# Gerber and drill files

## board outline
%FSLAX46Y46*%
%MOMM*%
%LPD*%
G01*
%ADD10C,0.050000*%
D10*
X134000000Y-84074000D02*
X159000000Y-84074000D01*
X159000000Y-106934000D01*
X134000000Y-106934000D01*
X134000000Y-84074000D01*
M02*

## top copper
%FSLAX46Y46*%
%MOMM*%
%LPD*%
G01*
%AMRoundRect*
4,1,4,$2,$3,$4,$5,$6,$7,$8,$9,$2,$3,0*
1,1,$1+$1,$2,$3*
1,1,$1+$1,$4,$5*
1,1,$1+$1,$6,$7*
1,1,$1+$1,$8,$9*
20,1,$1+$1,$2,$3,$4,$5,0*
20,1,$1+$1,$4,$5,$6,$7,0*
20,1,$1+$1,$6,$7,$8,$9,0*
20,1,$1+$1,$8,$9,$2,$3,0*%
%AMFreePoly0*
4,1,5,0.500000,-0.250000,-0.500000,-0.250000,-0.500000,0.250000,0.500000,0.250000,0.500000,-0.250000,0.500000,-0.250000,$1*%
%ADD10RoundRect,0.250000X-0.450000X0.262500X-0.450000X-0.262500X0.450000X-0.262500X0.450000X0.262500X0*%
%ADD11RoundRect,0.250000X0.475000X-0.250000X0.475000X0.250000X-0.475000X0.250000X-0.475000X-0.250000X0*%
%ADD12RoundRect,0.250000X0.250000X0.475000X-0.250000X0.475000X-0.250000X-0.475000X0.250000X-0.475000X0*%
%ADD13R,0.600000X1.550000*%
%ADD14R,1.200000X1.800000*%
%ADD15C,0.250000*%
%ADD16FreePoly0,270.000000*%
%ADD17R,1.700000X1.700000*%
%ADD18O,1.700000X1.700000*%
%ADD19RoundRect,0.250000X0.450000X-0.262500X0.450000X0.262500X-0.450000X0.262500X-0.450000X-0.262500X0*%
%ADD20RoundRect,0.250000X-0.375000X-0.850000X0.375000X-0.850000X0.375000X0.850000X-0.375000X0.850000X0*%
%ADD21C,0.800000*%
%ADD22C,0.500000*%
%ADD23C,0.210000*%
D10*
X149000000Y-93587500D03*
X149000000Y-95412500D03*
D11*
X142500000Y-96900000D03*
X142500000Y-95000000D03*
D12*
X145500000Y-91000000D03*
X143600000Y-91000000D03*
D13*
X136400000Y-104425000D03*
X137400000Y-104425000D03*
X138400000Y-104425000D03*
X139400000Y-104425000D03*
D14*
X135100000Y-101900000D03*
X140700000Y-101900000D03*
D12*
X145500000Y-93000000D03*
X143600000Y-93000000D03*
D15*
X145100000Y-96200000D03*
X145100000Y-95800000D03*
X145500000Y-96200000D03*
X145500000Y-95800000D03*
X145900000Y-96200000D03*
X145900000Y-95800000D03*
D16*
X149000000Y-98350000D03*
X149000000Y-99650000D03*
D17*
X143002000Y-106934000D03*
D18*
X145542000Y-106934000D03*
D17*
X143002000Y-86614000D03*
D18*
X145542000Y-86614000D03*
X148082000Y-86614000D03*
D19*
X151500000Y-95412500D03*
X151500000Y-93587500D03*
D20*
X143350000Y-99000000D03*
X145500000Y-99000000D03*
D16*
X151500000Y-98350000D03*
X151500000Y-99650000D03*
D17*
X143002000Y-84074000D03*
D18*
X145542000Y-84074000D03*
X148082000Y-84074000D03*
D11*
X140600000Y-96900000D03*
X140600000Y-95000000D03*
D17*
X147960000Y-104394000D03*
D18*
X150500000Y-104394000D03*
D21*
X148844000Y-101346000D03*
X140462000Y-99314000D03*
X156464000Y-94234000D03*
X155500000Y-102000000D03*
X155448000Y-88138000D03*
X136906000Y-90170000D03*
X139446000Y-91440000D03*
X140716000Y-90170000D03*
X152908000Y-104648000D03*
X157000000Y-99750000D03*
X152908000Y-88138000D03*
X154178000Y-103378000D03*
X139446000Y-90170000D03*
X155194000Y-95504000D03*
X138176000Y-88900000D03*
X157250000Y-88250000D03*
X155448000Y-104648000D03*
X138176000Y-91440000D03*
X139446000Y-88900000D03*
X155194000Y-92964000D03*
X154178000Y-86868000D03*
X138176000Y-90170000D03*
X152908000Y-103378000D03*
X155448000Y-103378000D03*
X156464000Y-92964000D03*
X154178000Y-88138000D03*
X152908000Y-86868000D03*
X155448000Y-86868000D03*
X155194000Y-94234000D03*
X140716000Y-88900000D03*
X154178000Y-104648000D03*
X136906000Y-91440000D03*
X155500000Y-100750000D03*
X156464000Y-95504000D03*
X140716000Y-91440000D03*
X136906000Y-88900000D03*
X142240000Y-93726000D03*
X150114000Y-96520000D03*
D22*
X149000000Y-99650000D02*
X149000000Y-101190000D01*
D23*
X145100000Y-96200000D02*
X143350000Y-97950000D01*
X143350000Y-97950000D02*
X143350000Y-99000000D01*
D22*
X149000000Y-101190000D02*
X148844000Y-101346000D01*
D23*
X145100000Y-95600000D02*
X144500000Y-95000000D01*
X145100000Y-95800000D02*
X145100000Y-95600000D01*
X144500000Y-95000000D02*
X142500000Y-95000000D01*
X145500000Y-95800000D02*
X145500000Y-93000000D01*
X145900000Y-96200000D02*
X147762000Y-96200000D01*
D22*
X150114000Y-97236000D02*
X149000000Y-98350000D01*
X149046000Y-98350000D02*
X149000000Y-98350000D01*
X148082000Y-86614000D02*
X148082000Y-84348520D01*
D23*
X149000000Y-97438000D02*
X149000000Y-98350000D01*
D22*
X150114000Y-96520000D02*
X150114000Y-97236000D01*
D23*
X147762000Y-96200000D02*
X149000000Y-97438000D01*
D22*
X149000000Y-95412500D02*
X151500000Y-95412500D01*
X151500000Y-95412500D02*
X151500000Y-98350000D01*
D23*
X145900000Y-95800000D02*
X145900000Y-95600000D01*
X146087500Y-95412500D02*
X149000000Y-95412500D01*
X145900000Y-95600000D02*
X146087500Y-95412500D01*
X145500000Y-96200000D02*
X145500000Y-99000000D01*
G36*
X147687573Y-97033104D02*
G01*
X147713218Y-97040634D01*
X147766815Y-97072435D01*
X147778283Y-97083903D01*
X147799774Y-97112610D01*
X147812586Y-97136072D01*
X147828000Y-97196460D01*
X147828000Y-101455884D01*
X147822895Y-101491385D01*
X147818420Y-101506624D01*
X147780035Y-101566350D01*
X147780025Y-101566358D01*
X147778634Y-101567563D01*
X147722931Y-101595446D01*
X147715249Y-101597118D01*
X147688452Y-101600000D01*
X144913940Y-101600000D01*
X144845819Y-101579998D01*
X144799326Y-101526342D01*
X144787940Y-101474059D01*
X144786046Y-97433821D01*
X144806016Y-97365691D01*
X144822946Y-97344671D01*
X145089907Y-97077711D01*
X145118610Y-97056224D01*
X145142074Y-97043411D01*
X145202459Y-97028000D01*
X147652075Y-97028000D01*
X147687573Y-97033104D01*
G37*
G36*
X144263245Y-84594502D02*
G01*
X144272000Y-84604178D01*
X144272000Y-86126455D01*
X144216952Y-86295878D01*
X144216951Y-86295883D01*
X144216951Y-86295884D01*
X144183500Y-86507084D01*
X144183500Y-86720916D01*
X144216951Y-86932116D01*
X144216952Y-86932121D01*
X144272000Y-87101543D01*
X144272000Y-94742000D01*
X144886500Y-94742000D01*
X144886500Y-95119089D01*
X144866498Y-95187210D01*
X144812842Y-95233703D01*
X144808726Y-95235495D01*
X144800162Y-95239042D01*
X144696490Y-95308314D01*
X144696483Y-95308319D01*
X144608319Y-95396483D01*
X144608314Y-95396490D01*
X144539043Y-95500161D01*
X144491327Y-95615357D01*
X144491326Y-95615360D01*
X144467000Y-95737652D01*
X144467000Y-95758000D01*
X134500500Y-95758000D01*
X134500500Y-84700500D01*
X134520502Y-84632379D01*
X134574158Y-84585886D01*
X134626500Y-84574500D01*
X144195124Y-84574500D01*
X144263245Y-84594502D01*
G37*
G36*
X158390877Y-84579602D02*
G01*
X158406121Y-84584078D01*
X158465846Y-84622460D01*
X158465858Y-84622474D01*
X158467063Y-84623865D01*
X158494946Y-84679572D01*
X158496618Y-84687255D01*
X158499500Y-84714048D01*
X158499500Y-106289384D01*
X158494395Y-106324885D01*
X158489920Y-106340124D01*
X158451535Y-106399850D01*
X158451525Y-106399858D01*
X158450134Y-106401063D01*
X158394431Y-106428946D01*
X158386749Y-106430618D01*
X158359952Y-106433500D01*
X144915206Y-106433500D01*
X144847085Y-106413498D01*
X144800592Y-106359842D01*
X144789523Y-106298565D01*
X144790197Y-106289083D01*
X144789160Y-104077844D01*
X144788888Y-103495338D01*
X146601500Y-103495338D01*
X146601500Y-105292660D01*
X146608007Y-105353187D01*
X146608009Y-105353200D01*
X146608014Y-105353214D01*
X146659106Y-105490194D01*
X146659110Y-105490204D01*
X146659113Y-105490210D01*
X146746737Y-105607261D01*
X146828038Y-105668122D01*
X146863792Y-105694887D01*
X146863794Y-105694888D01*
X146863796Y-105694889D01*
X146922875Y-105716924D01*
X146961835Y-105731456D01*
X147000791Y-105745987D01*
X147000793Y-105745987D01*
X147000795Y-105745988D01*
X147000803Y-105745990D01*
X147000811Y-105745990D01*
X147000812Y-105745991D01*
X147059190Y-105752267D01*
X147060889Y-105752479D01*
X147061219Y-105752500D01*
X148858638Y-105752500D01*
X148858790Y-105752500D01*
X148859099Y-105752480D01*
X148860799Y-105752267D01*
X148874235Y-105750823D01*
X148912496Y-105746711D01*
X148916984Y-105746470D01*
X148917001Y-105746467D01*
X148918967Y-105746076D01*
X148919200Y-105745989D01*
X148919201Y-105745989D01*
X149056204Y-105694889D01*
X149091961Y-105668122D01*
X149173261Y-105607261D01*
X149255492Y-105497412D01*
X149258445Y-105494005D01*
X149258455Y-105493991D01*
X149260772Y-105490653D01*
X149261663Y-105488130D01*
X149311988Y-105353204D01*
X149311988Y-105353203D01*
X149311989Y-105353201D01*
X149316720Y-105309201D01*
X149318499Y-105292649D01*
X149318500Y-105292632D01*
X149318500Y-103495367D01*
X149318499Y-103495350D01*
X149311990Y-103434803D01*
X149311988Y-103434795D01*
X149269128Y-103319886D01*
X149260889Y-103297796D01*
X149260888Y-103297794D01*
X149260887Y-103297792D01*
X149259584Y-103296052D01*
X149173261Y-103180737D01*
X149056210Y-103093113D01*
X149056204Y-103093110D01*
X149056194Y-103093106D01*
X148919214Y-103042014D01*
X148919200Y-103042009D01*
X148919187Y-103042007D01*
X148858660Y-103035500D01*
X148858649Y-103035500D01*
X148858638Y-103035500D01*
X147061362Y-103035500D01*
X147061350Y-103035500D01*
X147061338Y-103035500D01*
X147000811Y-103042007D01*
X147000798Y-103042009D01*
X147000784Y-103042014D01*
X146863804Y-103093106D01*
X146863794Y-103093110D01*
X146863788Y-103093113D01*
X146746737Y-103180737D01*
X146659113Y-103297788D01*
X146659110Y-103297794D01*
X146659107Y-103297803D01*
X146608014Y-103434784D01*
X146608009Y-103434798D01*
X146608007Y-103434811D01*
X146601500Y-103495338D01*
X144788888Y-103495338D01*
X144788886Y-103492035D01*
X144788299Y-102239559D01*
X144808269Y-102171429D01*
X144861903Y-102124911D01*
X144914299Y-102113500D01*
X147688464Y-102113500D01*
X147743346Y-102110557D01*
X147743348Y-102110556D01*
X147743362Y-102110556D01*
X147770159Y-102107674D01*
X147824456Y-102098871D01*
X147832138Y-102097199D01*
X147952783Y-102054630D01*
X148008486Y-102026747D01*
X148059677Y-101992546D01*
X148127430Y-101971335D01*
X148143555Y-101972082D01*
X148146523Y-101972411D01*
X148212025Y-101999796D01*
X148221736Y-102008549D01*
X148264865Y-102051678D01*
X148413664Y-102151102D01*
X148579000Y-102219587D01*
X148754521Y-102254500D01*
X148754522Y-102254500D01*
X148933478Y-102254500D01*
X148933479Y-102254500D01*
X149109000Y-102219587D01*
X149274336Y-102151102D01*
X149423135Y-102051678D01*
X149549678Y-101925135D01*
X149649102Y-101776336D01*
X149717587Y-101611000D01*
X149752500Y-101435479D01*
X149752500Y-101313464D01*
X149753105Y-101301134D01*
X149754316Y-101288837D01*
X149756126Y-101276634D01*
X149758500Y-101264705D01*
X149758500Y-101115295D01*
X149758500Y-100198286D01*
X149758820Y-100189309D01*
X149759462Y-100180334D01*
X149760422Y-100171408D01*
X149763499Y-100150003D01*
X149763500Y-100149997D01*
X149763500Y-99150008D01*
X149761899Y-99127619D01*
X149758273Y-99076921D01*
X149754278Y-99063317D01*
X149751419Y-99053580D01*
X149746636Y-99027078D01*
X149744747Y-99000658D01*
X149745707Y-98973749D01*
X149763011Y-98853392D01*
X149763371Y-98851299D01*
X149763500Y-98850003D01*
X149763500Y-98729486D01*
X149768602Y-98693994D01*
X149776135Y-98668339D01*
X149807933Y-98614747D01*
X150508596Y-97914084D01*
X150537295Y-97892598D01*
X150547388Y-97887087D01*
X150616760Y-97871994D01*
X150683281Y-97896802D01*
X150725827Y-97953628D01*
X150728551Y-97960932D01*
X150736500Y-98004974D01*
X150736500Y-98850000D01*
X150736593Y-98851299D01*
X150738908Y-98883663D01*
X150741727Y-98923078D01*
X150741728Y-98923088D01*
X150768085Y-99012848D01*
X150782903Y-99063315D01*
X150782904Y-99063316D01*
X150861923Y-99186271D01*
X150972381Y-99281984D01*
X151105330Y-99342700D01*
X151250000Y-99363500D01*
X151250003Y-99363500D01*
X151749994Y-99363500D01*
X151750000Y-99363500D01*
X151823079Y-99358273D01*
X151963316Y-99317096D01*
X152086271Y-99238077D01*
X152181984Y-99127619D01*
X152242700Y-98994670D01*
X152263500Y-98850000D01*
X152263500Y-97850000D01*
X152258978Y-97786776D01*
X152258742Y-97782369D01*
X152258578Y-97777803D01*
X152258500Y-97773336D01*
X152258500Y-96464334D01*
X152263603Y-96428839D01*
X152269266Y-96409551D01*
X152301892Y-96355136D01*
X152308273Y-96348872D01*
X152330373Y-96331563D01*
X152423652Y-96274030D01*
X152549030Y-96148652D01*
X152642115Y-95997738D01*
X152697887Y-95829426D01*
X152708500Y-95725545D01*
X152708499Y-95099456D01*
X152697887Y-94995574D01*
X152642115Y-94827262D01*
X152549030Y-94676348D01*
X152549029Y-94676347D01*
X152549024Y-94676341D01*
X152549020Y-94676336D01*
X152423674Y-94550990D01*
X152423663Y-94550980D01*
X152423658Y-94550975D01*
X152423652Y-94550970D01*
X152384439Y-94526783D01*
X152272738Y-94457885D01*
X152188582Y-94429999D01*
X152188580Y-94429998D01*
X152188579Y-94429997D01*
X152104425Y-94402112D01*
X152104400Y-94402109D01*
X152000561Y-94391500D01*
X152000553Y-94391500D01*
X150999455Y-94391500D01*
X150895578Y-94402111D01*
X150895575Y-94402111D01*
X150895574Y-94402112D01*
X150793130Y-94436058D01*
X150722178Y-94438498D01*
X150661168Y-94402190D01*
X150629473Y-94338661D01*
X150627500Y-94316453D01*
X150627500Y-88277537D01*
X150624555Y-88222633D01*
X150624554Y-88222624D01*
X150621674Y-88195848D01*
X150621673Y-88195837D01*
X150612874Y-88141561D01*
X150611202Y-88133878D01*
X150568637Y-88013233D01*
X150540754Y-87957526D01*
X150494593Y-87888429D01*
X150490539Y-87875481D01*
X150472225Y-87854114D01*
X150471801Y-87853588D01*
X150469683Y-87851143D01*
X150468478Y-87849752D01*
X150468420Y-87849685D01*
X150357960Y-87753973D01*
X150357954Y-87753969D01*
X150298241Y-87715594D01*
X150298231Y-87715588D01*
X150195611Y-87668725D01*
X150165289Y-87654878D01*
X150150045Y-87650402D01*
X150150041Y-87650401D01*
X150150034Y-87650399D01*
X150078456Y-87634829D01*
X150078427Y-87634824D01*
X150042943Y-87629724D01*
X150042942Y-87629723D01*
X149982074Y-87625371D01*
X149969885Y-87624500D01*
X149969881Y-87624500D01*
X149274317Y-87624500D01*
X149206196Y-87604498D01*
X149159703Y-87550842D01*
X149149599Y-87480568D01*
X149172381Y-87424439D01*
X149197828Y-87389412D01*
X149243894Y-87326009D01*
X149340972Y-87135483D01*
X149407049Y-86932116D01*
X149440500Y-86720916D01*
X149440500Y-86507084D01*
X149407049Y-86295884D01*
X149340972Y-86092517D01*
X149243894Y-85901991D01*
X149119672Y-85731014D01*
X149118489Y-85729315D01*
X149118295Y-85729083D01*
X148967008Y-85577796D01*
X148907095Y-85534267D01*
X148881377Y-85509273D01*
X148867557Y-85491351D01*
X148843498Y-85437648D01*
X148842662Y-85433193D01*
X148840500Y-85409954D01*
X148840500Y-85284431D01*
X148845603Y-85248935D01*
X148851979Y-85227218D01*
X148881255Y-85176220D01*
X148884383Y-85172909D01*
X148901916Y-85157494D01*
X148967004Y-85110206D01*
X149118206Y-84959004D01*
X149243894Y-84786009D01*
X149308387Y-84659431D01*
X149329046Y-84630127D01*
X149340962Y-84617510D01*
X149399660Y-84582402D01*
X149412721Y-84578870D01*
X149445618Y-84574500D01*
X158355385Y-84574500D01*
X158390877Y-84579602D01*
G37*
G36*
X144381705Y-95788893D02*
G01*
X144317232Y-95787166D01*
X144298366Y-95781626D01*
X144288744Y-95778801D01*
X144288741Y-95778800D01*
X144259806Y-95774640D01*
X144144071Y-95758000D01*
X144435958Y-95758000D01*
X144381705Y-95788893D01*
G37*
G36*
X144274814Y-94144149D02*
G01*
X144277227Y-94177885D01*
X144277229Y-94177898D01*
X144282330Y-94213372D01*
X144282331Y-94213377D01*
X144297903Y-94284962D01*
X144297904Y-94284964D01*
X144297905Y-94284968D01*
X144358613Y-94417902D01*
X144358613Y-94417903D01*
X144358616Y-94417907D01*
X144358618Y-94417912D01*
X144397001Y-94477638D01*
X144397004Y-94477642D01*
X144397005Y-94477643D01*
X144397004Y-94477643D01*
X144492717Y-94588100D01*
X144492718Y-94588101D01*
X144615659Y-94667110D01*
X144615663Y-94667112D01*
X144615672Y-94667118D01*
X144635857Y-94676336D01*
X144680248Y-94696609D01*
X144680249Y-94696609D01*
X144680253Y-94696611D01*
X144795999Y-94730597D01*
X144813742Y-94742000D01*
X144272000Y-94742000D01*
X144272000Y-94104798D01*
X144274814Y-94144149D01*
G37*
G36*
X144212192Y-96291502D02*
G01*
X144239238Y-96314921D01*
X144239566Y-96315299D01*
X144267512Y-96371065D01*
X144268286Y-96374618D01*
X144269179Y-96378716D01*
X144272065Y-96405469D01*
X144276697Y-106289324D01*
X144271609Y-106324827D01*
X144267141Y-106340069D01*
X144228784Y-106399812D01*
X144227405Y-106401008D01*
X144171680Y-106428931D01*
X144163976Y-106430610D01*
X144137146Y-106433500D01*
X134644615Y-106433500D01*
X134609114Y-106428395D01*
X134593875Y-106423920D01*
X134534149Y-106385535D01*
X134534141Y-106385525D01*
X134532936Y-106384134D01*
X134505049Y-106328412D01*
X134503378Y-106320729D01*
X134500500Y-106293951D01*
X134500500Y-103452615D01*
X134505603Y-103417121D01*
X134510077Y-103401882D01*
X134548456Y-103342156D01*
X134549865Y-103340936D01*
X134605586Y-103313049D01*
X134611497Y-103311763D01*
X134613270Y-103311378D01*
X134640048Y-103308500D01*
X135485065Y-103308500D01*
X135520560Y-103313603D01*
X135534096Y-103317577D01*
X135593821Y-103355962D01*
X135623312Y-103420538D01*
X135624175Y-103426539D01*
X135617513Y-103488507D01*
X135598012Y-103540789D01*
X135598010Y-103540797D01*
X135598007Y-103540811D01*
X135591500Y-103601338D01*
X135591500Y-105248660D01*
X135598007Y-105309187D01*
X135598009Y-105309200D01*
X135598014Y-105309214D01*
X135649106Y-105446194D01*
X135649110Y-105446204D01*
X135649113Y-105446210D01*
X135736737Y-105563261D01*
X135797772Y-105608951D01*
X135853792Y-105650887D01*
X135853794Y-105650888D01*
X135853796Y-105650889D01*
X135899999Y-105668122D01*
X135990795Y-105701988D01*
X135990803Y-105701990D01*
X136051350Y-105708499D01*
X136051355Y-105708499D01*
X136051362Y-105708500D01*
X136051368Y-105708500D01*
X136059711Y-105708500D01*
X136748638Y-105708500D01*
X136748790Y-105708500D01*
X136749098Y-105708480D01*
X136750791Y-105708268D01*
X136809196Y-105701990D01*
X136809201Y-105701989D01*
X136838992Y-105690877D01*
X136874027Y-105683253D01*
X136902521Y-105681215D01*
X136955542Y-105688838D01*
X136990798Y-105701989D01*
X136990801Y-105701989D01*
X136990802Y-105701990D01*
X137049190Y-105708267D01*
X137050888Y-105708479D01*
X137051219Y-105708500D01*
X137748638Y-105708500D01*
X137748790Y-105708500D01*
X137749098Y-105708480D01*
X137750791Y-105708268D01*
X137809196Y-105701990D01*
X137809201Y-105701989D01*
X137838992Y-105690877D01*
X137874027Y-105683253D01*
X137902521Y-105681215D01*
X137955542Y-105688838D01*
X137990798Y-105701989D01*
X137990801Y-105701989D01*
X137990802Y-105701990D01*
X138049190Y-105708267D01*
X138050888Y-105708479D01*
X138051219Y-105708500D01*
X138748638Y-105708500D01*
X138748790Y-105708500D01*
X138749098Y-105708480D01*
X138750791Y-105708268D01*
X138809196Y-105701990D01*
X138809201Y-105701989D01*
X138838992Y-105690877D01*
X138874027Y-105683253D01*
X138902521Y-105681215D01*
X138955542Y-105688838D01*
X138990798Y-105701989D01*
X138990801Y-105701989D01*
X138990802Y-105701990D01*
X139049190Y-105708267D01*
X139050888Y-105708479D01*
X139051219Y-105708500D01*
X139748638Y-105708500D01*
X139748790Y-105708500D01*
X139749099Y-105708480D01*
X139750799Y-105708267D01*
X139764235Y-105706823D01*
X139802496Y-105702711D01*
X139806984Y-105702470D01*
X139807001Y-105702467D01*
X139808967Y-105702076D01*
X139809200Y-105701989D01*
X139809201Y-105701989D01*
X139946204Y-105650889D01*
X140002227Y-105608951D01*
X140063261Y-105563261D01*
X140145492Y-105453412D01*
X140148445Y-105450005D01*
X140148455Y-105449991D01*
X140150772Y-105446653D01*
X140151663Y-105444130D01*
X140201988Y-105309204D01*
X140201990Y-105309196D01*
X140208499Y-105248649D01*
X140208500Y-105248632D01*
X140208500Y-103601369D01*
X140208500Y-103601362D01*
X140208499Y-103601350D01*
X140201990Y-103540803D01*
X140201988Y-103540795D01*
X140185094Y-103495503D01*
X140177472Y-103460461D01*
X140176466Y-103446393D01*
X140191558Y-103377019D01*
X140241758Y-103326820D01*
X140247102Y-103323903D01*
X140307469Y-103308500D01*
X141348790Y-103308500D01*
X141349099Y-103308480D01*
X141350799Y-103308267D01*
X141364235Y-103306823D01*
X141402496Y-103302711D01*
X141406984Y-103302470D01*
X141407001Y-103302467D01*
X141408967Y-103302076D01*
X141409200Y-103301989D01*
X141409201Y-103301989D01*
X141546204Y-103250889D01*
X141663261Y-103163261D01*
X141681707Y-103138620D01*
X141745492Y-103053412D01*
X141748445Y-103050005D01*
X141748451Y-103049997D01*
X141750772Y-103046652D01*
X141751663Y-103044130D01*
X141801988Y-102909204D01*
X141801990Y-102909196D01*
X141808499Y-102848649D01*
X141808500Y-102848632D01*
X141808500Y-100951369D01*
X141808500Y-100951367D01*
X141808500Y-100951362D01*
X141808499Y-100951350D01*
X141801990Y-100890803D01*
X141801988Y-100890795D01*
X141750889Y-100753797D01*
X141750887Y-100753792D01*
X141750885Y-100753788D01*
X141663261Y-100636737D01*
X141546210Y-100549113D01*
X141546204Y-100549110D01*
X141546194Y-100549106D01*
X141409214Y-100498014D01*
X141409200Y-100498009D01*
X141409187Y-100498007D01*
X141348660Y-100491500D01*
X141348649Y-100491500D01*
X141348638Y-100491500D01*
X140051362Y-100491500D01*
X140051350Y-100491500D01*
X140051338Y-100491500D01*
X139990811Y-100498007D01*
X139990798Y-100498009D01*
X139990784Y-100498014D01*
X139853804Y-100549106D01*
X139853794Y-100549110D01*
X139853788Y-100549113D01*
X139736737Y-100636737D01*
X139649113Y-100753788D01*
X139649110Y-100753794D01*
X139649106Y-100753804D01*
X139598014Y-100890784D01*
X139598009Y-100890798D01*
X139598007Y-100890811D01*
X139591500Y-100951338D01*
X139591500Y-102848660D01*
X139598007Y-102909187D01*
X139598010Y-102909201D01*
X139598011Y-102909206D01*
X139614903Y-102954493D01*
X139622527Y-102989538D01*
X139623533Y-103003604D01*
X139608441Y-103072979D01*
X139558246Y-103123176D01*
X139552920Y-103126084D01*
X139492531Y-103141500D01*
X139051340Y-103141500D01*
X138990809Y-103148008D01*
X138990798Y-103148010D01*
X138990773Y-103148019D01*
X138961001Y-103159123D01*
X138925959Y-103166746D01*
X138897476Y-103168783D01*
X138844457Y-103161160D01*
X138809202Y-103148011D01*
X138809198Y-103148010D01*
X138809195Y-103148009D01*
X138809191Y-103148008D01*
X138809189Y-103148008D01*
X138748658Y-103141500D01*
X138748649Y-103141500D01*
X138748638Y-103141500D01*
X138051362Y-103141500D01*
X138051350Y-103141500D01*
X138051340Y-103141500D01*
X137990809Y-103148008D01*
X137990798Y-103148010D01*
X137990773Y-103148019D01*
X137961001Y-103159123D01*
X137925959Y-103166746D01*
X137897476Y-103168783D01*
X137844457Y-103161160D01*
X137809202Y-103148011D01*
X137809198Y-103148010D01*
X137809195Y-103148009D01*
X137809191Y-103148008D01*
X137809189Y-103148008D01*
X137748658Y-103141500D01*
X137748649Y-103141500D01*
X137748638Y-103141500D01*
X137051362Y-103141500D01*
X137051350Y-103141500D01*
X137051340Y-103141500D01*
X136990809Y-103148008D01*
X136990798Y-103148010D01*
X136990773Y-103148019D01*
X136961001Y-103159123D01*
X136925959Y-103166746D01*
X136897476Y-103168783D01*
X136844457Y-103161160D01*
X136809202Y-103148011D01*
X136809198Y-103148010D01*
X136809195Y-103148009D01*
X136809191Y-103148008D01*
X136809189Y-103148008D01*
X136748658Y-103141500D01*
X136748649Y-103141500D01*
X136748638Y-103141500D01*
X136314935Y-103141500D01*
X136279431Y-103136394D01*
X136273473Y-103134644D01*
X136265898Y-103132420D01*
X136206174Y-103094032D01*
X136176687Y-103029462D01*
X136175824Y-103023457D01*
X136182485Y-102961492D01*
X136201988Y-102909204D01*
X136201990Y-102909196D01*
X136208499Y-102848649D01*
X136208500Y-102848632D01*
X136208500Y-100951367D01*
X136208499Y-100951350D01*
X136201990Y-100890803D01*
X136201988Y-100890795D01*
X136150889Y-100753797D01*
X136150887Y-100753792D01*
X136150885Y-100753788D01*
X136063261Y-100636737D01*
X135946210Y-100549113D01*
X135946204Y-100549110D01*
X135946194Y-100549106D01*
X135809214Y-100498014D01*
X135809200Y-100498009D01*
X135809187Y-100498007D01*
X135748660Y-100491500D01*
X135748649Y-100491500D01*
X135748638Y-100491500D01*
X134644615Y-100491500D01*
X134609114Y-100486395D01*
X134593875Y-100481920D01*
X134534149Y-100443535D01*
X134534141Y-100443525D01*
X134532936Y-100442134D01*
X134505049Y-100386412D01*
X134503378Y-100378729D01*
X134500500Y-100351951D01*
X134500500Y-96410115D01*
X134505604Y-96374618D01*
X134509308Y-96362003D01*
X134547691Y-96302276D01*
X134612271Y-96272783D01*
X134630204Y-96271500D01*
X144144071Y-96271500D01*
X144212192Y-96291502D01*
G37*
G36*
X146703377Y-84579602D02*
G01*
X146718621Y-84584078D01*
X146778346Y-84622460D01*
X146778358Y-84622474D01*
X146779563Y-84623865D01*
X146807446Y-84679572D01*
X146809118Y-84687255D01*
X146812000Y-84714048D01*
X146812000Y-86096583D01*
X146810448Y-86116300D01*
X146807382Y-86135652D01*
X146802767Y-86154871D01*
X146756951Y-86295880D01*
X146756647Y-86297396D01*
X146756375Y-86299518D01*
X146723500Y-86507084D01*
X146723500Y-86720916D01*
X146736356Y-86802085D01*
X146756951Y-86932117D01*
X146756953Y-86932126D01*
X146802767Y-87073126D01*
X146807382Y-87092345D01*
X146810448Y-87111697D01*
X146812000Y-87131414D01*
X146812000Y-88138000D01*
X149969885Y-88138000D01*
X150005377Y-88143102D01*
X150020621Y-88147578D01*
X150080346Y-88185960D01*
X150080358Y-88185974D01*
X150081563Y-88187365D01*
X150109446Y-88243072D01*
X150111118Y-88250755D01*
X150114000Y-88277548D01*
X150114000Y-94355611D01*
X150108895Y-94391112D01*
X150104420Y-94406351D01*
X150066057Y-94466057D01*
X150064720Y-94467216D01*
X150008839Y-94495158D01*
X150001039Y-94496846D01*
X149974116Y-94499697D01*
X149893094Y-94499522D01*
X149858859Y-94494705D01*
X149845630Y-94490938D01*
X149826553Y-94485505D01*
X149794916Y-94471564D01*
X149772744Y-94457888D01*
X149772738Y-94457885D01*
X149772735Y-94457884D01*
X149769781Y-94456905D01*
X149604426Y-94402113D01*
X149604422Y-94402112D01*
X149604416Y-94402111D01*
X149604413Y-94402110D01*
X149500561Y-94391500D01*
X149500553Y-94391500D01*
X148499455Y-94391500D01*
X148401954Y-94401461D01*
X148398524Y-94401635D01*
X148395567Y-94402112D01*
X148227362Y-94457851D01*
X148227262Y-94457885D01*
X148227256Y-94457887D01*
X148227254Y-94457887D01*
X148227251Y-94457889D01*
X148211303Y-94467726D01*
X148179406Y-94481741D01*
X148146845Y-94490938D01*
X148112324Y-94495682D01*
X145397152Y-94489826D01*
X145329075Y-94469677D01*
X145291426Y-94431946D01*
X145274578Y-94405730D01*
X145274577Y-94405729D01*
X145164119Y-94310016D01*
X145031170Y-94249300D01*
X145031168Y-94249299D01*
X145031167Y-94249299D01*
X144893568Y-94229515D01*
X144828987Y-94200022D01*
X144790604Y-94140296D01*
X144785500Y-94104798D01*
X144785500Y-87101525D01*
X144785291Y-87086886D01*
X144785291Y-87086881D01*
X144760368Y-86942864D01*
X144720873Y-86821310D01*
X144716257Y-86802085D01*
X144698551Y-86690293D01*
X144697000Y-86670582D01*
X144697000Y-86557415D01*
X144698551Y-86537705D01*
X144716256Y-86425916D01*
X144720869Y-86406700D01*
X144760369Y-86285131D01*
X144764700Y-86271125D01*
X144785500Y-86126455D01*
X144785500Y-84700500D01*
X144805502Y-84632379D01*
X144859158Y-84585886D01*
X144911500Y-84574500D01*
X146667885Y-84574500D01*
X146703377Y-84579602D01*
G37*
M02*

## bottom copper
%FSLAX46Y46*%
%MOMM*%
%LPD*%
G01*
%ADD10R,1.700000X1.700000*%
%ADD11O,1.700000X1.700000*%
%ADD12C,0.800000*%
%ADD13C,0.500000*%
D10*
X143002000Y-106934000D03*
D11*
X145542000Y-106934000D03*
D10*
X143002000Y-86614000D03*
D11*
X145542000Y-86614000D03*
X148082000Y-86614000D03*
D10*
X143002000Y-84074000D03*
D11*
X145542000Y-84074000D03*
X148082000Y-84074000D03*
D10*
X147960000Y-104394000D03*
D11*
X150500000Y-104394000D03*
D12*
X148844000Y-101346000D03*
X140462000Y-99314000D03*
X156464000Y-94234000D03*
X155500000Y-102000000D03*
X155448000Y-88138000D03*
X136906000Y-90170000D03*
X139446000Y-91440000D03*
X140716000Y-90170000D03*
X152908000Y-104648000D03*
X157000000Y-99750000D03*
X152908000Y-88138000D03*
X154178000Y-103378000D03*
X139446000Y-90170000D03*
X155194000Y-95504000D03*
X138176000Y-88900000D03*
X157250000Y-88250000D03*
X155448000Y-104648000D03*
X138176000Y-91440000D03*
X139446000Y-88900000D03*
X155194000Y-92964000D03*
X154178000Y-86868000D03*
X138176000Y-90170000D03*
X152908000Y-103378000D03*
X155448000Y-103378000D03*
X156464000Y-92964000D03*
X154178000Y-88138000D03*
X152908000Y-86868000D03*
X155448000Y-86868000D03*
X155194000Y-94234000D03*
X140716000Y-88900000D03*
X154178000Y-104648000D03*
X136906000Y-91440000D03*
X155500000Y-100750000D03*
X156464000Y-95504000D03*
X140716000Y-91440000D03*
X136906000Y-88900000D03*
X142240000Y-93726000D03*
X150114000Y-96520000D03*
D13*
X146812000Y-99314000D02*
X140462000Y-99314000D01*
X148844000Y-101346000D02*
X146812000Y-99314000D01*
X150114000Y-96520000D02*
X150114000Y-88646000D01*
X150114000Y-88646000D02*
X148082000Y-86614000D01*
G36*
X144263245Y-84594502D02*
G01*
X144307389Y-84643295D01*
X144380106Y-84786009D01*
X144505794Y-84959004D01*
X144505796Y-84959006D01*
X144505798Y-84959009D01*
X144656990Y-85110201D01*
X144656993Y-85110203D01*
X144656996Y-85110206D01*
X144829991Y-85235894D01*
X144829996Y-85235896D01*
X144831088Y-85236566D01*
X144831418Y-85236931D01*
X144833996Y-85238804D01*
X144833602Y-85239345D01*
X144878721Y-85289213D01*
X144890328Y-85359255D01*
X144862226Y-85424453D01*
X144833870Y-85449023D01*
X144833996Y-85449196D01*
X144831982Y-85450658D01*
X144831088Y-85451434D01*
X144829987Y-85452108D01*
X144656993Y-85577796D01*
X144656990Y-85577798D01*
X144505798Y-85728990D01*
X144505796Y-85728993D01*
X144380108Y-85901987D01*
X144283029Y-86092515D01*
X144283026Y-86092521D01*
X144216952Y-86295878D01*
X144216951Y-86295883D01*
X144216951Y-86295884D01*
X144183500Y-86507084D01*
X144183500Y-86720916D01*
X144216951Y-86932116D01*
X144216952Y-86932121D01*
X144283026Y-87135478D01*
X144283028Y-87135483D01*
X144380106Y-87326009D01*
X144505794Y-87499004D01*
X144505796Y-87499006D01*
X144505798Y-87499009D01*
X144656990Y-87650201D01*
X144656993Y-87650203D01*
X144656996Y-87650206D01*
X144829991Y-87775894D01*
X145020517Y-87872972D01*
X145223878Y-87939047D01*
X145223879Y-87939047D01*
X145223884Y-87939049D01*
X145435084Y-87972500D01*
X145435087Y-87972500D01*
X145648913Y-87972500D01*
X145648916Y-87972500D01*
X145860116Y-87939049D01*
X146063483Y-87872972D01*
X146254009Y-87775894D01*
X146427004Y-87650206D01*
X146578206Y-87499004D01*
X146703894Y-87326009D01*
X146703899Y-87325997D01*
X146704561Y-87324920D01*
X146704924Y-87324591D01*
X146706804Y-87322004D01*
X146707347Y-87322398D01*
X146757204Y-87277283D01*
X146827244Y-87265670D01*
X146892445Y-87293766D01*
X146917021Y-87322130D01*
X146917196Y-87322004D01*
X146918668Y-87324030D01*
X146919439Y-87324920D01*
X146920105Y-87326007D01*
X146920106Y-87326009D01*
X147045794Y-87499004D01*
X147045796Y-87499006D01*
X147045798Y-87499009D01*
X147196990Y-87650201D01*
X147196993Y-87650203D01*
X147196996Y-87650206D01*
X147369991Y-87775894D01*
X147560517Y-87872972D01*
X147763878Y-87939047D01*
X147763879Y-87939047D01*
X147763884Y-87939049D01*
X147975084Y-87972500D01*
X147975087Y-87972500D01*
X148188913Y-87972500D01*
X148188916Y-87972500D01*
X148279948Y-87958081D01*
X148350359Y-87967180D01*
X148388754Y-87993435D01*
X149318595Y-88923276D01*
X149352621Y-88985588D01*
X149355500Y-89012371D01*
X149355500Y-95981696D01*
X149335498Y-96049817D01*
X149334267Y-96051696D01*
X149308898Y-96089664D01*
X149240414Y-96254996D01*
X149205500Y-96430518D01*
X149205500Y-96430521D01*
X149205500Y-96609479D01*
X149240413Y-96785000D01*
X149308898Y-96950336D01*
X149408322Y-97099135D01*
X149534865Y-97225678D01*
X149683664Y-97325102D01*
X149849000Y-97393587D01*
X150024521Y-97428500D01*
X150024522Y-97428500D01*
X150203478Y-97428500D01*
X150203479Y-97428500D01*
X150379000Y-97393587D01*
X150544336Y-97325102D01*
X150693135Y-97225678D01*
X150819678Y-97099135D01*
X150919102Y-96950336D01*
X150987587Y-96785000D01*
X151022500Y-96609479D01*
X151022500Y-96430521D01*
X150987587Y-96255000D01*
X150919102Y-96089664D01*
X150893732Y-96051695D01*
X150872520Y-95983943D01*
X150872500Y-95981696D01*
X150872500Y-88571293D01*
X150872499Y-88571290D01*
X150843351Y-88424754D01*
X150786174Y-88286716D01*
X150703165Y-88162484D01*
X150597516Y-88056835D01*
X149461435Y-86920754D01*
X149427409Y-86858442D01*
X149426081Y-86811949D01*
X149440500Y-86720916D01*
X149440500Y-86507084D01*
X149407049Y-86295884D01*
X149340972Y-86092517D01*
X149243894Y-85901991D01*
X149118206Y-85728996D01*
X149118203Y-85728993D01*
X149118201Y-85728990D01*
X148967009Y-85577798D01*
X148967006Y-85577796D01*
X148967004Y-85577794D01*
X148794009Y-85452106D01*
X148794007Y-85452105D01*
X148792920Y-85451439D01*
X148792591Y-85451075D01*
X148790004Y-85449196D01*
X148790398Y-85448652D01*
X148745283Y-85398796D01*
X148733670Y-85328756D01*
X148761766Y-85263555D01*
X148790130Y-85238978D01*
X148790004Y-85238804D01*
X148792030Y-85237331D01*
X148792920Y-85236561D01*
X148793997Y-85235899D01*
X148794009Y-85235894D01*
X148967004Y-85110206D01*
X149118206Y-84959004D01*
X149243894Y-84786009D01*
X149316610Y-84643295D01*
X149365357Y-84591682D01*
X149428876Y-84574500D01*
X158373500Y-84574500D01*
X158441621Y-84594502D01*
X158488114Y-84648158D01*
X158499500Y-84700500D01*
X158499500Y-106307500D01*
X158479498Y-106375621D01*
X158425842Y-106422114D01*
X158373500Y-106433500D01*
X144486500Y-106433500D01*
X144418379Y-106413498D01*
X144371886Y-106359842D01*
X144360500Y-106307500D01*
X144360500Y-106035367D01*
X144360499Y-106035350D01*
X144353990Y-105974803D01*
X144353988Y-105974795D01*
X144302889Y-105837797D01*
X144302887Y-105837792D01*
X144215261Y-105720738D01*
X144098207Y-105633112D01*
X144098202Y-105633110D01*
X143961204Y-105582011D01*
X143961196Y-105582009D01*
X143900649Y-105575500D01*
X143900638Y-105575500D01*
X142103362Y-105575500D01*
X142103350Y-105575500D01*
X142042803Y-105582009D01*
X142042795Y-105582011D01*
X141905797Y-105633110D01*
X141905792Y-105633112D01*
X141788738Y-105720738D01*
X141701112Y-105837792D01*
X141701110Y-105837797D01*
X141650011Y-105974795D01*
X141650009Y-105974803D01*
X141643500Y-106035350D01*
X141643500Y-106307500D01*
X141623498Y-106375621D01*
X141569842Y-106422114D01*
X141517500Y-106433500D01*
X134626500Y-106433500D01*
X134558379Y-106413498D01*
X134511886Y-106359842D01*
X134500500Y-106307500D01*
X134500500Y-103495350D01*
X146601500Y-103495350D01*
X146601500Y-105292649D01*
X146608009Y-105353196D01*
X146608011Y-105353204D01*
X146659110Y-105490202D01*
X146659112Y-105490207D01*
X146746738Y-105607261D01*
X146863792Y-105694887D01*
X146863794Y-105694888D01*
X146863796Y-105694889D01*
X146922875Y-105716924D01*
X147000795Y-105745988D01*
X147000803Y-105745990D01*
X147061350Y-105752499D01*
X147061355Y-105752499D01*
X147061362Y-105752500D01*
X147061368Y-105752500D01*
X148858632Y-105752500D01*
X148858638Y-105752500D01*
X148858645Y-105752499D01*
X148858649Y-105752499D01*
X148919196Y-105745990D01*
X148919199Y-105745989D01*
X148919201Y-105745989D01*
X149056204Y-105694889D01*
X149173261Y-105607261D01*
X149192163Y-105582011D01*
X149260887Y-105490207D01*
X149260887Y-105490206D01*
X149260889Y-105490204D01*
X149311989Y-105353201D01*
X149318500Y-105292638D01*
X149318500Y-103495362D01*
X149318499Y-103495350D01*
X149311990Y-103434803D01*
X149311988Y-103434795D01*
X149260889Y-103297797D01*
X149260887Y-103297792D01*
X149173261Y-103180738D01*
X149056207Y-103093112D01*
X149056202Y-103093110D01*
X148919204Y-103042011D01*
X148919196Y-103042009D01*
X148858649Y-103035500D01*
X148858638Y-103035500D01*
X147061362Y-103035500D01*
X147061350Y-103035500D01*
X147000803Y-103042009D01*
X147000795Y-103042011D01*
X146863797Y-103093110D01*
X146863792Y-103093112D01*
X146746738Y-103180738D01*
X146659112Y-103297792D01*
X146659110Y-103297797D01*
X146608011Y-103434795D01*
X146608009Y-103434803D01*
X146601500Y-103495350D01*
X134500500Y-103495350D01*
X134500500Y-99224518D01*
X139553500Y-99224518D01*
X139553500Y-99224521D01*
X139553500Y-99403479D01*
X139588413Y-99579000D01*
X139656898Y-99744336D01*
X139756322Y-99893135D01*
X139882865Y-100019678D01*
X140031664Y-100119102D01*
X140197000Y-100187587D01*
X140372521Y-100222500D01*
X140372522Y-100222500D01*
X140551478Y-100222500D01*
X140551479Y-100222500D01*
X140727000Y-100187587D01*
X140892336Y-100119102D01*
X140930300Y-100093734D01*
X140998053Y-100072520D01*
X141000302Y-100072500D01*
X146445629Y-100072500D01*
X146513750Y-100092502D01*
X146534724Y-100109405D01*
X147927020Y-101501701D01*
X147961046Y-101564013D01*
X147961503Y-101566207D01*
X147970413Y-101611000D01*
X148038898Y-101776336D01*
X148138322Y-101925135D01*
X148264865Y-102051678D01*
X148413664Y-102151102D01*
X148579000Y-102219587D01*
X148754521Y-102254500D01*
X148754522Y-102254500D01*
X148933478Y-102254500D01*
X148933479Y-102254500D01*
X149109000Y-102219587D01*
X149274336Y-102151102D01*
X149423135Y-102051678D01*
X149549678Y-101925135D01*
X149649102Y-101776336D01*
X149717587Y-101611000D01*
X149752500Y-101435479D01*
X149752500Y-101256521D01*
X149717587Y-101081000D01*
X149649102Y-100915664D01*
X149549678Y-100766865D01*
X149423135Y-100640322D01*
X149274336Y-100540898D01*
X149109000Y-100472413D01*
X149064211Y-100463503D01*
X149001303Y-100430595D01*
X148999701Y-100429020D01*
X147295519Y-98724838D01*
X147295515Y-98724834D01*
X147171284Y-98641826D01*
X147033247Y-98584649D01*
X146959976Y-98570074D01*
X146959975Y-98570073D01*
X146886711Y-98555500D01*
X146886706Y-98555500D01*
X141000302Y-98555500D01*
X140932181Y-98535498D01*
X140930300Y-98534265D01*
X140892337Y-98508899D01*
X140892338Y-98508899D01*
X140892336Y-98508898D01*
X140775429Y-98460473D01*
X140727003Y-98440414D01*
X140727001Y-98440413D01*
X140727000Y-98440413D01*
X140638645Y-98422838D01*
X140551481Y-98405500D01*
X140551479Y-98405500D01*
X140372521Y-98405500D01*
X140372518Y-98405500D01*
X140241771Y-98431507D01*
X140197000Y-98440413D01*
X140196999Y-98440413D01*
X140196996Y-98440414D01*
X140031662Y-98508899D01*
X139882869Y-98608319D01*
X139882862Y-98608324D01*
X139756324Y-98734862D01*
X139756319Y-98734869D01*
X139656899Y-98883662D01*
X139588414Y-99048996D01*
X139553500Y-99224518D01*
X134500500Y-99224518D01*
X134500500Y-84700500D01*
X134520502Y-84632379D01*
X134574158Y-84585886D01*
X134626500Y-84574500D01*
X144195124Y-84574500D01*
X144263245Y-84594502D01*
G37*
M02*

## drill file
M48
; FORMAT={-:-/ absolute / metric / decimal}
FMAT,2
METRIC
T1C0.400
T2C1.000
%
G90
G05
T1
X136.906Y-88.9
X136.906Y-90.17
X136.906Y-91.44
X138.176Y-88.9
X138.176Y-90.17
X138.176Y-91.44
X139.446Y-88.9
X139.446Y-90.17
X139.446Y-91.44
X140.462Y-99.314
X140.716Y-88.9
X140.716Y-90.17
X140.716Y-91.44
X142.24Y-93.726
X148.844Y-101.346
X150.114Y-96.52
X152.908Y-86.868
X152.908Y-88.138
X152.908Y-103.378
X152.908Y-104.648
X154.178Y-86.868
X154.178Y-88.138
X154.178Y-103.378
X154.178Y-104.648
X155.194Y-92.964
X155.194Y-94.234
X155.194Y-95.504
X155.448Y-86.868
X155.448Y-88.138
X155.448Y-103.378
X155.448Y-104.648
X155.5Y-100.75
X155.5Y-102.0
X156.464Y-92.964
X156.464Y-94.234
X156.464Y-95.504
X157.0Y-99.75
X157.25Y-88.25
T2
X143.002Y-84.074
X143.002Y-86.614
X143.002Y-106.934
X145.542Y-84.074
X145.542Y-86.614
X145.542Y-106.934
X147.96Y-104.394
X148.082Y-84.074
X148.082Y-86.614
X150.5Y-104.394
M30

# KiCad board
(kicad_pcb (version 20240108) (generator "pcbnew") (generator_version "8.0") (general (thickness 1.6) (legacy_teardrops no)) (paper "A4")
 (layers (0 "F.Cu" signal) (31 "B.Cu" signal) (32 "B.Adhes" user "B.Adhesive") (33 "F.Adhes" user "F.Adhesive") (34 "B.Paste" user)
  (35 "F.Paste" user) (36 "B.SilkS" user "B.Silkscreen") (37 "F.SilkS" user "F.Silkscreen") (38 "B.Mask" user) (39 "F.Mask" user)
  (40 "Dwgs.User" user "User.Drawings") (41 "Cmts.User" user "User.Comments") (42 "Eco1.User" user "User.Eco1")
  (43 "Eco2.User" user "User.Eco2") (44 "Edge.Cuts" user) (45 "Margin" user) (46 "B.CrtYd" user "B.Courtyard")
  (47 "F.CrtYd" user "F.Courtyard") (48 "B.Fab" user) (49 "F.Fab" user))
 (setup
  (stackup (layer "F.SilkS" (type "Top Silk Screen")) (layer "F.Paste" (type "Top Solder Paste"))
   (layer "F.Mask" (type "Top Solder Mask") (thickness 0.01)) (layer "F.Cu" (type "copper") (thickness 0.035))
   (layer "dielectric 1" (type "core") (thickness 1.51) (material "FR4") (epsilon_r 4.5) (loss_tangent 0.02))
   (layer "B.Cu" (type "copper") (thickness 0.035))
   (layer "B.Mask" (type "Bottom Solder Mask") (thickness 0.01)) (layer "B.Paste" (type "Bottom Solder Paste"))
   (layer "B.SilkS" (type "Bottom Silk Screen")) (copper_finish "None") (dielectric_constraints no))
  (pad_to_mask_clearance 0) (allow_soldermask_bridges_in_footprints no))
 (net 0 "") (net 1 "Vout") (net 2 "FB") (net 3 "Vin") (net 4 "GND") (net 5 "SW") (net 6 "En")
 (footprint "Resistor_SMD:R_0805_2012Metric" (layer "F.Cu") (at 149 94.5 -90)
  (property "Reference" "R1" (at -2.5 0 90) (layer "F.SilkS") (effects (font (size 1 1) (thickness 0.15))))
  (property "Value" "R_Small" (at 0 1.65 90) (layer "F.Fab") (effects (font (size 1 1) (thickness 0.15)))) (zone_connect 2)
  (pad "1" smd roundrect (at -0.9125 0 270) (size 1.025 1.4) (layers "F.Cu" "F.Paste" "F.Mask") (roundrect_rratio 0.243902) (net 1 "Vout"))
  (pad "2" smd roundrect (at 0.9125 0 270) (size 1.025 1.4) (layers "F.Cu" "F.Paste" "F.Mask") (roundrect_rratio 0.243902) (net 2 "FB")))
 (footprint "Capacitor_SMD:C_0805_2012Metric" (layer "F.Cu") (at 142.5 95.95 90)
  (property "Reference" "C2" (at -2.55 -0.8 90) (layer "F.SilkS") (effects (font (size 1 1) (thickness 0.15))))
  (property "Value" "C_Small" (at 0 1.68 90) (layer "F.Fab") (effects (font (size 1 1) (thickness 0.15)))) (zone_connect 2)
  (pad "1" smd roundrect (at -0.95 0 90) (size 1 1.45) (layers "F.Cu" "F.Paste" "F.Mask") (roundrect_rratio 0.25) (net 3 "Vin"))
  (pad "2" smd roundrect (at 0.95 0 90) (size 1 1.45) (layers "F.Cu" "F.Paste" "F.Mask") (roundrect_rratio 0.25) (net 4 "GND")))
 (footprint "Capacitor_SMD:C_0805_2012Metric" (layer "F.Cu") (at 144.55 91 180)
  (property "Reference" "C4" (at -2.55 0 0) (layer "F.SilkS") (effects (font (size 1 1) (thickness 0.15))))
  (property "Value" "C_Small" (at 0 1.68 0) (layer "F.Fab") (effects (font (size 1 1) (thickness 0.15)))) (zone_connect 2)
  (pad "1" smd roundrect (at -0.95 0 180) (size 1 1.45) (layers "F.Cu" "F.Paste" "F.Mask") (roundrect_rratio 0.25) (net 1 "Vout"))
  (pad "2" smd roundrect (at 0.95 0 180) (size 1 1.45) (layers "F.Cu" "F.Paste" "F.Mask") (roundrect_rratio 0.25) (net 4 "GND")))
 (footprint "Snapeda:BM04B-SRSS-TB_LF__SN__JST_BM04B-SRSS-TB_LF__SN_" (layer "F.Cu") (at 137.9 101.9)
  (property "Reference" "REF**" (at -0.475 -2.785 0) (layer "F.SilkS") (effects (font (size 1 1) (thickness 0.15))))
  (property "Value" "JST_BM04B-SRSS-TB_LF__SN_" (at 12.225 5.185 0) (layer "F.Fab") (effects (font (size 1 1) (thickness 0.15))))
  (pad "1" smd rect (at -1.5 2.525) (size 0.6 1.55) (layers "F.Cu" "F.Paste" "F.Mask") (solder_mask_margin 0.102))
  (pad "2" smd rect (at -0.5 2.525) (size 0.6 1.55) (layers "F.Cu" "F.Paste" "F.Mask") (solder_mask_margin 0.102))
  (pad "3" smd rect (at 0.5 2.525) (size 0.6 1.55) (layers "F.Cu" "F.Paste" "F.Mask") (solder_mask_margin 0.102))
  (pad "4" smd rect (at 1.5 2.525) (size 0.6 1.55) (layers "F.Cu" "F.Paste" "F.Mask") (solder_mask_margin 0.102))
  (pad "S1" smd rect (at -2.8 0) (size 1.2 1.8) (layers "F.Cu" "F.Paste" "F.Mask") (solder_mask_margin 0.102))
  (pad "S2" smd rect (at 2.8 0) (size 1.2 1.8) (layers "F.Cu" "F.Paste" "F.Mask") (solder_mask_margin 0.102)))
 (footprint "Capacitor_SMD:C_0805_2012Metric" (layer "F.Cu") (at 144.55 93 180)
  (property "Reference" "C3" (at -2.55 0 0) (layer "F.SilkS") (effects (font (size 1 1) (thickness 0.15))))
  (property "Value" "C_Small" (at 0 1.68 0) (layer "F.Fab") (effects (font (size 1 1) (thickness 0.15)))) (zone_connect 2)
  (pad "1" smd roundrect (at -0.95 0 180) (size 1 1.45) (layers "F.Cu" "F.Paste" "F.Mask") (roundrect_rratio 0.25) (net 1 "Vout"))
  (pad "2" smd roundrect (at 0.95 0 180) (size 1 1.45) (layers "F.Cu" "F.Paste" "F.Mask") (roundrect_rratio 0.25) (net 4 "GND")))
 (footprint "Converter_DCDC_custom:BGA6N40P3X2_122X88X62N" (layer "F.Cu") (at 145.5 96 90)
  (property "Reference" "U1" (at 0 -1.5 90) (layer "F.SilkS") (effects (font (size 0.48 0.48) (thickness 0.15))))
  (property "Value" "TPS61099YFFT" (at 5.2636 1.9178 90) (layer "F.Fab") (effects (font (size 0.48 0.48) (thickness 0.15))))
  (pad "A1" smd circle (at -0.2 -0.4 90) (size 0.25 0.25) (layers "F.Cu" "F.Paste" "F.Mask") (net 3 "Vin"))
  (pad "A2" smd circle (at 0.2 -0.4 90) (size 0.25 0.25) (layers "F.Cu" "F.Paste" "F.Mask") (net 4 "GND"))
  (pad "B1" smd circle (at -0.2 0 90) (size 0.25 0.25) (layers "F.Cu" "F.Paste" "F.Mask") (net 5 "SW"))
  (pad "B2" smd circle (at 0.2 0 90) (size 0.25 0.25) (layers "F.Cu" "F.Paste" "F.Mask") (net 1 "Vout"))
  (pad "C1" smd circle (at -0.2 0.4 90) (size 0.25 0.25) (layers "F.Cu" "F.Paste" "F.Mask") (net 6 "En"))
  (pad "C2" smd circle (at 0.2 0.4 90) (size 0.25 0.25) (layers "F.Cu" "F.Paste" "F.Mask") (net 2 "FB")))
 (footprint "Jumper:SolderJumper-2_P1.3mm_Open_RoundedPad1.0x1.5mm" (layer "F.Cu") (at 149 99 -90)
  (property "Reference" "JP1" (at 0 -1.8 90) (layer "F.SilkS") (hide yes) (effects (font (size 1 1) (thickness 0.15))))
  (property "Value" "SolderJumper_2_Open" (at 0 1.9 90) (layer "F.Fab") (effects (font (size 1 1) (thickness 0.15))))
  (pad "1" smd custom (at -0.65 0 270) (size 1 0.5) (layers "F.Cu" "F.Mask") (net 6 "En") (zone_connect 2)
   (options (clearance outline) (anchor rect)) (primitives))
  (pad "2" smd custom (at 0.65 0 270) (size 1 0.5) (layers "F.Cu" "F.Mask") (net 3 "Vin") (zone_connect 2)
   (options (clearance outline) (anchor rect)) (primitives)))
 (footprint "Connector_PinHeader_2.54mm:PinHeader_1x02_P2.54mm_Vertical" (layer "F.Cu") (at 143.002 106.934 90)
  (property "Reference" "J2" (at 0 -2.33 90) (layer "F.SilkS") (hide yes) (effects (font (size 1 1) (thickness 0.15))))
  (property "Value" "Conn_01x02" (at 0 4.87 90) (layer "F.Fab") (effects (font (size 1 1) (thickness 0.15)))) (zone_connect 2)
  (pad "1" thru_hole rect (at 0 0 90) (size 1.7 1.7) (drill 1) (layers "*.Cu" "*.Mask") (remove_unused_layers no) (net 3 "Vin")
   (zone_connect 2))
  (pad "2" thru_hole oval (at 0 2.54 90) (size 1.7 1.7) (drill 1) (layers "*.Cu" "*.Mask") (remove_unused_layers no) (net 4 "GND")
   (zone_connect 2)))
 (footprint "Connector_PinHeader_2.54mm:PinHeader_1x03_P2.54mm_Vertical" (layer "F.Cu") (at 143.002 86.614 90)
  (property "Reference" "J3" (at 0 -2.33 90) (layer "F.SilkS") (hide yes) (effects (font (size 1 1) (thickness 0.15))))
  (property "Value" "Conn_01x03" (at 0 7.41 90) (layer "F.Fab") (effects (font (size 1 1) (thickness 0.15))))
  (pad "1" thru_hole rect (at 0 0 90) (size 1.7 1.7) (drill 1) (layers "*.Cu" "*.Mask") (remove_unused_layers no) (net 4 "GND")
   (zone_connect 2))
  (pad "2" thru_hole oval (at 0 2.54 90) (size 1.7 1.7) (drill 1) (layers "*.Cu" "*.Mask") (remove_unused_layers no) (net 1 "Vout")
   (zone_connect 2))
  (pad "3" thru_hole oval (at 0 5.08 90) (size 1.7 1.7) (drill 1) (layers "*.Cu" "*.Mask") (remove_unused_layers no) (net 6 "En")))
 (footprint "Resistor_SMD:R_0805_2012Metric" (layer "F.Cu") (at 151.5 94.5 90)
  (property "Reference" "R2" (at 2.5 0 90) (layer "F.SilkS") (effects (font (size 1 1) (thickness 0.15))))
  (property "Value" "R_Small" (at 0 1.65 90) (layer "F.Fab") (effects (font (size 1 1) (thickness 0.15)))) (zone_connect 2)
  (pad "1" smd roundrect (at -0.9125 0 90) (size 1.025 1.4) (layers "F.Cu" "F.Paste" "F.Mask") (roundrect_rratio 0.243902) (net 2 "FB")
   (zone_connect 2))
  (pad "2" smd roundrect (at 0.9125 0 90) (size 1.025 1.4) (layers "F.Cu" "F.Paste" "F.Mask") (roundrect_rratio 0.243902) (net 4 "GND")
   (zone_connect 2)))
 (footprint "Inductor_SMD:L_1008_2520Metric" (layer "F.Cu") (at 144.425 99)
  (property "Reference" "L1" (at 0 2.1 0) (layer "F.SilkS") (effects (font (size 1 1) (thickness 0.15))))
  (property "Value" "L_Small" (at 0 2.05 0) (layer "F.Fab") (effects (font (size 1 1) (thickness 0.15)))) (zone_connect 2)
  (pad "1" smd roundrect (at -1.075 0) (size 1.25 2.2) (layers "F.Cu" "F.Paste" "F.Mask") (roundrect_rratio 0.2) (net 3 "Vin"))
  (pad "2" smd roundrect (at 1.075 0) (size 1.25 2.2) (layers "F.Cu" "F.Paste" "F.Mask") (roundrect_rratio 0.2) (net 5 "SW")))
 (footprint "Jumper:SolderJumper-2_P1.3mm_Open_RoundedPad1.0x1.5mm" (layer "F.Cu") (at 151.5 99 -90)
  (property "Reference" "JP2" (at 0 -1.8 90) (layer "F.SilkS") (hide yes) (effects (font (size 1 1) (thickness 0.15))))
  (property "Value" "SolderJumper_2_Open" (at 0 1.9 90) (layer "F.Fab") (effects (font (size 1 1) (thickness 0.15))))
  (pad "1" smd custom (at -0.65 0 270) (size 1 0.5) (layers "F.Cu" "F.Mask") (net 2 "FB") (zone_connect 2)
   (options (clearance outline) (anchor rect)) (primitives))
  (pad "2" smd custom (at 0.65 0 270) (size 1 0.5) (layers "F.Cu" "F.Mask") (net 4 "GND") (zone_connect 2)
   (options (clearance outline) (anchor rect)) (primitives)))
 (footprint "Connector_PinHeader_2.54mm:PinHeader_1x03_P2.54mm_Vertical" (layer "F.Cu") (at 143.002 84.074 90)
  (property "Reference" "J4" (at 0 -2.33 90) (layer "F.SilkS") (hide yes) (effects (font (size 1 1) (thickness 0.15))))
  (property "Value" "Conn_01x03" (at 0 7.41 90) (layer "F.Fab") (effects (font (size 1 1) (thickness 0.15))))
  (pad "1" thru_hole rect (at 0 0 90) (size 1.7 1.7) (drill 1) (layers "*.Cu" "*.Mask") (remove_unused_layers no) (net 4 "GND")
   (zone_connect 2))
  (pad "2" thru_hole oval (at 0 2.54 90) (size 1.7 1.7) (drill 1) (layers "*.Cu" "*.Mask") (remove_unused_layers no) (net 1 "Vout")
   (zone_connect 2))
  (pad "3" thru_hole oval (at 0 5.08 90) (size 1.7 1.7) (drill 1) (layers "*.Cu" "*.Mask") (remove_unused_layers no) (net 6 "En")))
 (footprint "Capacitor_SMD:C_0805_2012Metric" (layer "F.Cu") (at 140.6 95.95 90)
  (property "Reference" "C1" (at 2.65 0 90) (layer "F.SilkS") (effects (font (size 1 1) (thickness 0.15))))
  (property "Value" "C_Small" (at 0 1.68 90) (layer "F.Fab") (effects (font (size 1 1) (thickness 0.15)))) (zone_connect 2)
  (pad "1" smd roundrect (at -0.95 0 90) (size 1 1.45) (layers "F.Cu" "F.Paste" "F.Mask") (roundrect_rratio 0.25) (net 3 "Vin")
   (zone_connect 2))
  (pad "2" smd roundrect (at 0.95 0 90) (size 1 1.45) (layers "F.Cu" "F.Paste" "F.Mask") (roundrect_rratio 0.25) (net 4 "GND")
   (zone_connect 2)))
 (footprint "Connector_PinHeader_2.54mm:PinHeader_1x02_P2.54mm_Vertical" (layer "F.Cu") (at 147.96 104.394 90)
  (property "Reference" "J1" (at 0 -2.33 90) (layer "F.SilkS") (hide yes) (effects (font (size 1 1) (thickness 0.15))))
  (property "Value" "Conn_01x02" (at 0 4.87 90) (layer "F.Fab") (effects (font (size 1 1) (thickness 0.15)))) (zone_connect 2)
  (pad "1" thru_hole rect (at 0 0 90) (size 1.7 1.7) (drill 1) (layers "*.Cu" "*.Mask") (remove_unused_layers no) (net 3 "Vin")
   (zone_connect 2))
  (pad "2" thru_hole oval (at 0 2.54 90) (size 1.7 1.7) (drill 1) (layers "*.Cu" "*.Mask") (remove_unused_layers no) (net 4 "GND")
   (zone_connect 2)))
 (gr_rect (start 134 84.074) (end 159 106.934) (stroke (width 0.05) (type solid)) (fill none) (layer "Edge.Cuts"))
 (segment (start 149 99.65) (end 149 101.19) (width 0.5) (layer "F.Cu") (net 3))
 (segment (start 145.1 96.2) (end 143.35 97.95) (width 0.21) (layer "F.Cu") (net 3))
 (segment (start 143.35 97.95) (end 143.35 99) (width 0.21) (layer "F.Cu") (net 3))
 (segment (start 149 101.19) (end 148.844 101.346) (width 0.5) (layer "F.Cu") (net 3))
 (via (at 148.844 101.346) (size 0.8) (drill 0.4) (layers "F.Cu" "B.Cu") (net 3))
 (via (at 140.462 99.314) (size 0.8) (drill 0.4) (layers "F.Cu" "B.Cu") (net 3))
 (segment (start 146.812 99.314) (end 140.462 99.314) (width 0.5) (layer "B.Cu") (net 3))
 (segment (start 148.844 101.346) (end 146.812 99.314) (width 0.5) (layer "B.Cu") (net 3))
 (segment (start 145.1 95.6) (end 144.5 95) (width 0.21) (layer "F.Cu") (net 4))
 (segment (start 145.1 95.8) (end 145.1 95.6) (width 0.21) (layer "F.Cu") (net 4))
 (segment (start 144.5 95) (end 142.5 95) (width 0.21) (layer "F.Cu") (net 4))
 (via (at 156.464 94.234) (size 0.8) (drill 0.4) (layers "F.Cu" "B.Cu") (free yes) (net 4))
 (via (at 155.5 102) (size 0.8) (drill 0.4) (layers "F.Cu" "B.Cu") (free yes) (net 4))
 (via (at 155.448 88.138) (size 0.8) (drill 0.4) (layers "F.Cu" "B.Cu") (free yes) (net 4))
 (via (at 136.906 90.17) (size 0.8) (drill 0.4) (layers "F.Cu" "B.Cu") (free yes) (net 4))
 (via (at 139.446 91.44) (size 0.8) (drill 0.4) (layers "F.Cu" "B.Cu") (free yes) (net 4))
 (via (at 140.716 90.17) (size 0.8) (drill 0.4) (layers "F.Cu" "B.Cu") (free yes) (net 4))
 (via (at 152.908 104.648) (size 0.8) (drill 0.4) (layers "F.Cu" "B.Cu") (free yes) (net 4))
 (via (at 157 99.75) (size 0.8) (drill 0.4) (layers "F.Cu" "B.Cu") (free yes) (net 4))
 (via (at 152.908 88.138) (size 0.8) (drill 0.4) (layers "F.Cu" "B.Cu") (free yes) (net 4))
 (via (at 154.178 103.378) (size 0.8) (drill 0.4) (layers "F.Cu" "B.Cu") (free yes) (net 4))
 (via (at 139.446 90.17) (size 0.8) (drill 0.4) (layers "F.Cu" "B.Cu") (free yes) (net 4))
 (via (at 155.194 95.504) (size 0.8) (drill 0.4) (layers "F.Cu" "B.Cu") (free yes) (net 4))
 (via (at 138.176 88.9) (size 0.8) (drill 0.4) (layers "F.Cu" "B.Cu") (free yes) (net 4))
 (via (at 157.25 88.25) (size 0.8) (drill 0.4) (layers "F.Cu" "B.Cu") (free yes) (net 4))
 (via (at 155.448 104.648) (size 0.8) (drill 0.4) (layers "F.Cu" "B.Cu") (free yes) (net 4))
 (via (at 138.176 91.44) (size 0.8) (drill 0.4) (layers "F.Cu" "B.Cu") (free yes) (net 4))
 (via (at 139.446 88.9) (size 0.8) (drill 0.4) (layers "F.Cu" "B.Cu") (free yes) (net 4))
 (via (at 155.194 92.964) (size 0.8) (drill 0.4) (layers "F.Cu" "B.Cu") (free yes) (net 4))
 (via (at 154.178 86.868) (size 0.8) (drill 0.4) (layers "F.Cu" "B.Cu") (free yes) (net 4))
 (via (at 138.176 90.17) (size 0.8) (drill 0.4) (layers "F.Cu" "B.Cu") (free yes) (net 4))
 (via (at 152.908 103.378) (size 0.8) (drill 0.4) (layers "F.Cu" "B.Cu") (free yes) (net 4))
 (via (at 155.448 103.378) (size 0.8) (drill 0.4) (layers "F.Cu" "B.Cu") (free yes) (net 4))
 (via (at 156.464 92.964) (size 0.8) (drill 0.4) (layers "F.Cu" "B.Cu") (free yes) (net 4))
 (via (at 154.178 88.138) (size 0.8) (drill 0.4) (layers "F.Cu" "B.Cu") (free yes) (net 4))
 (via (at 152.908 86.868) (size 0.8) (drill 0.4) (layers "F.Cu" "B.Cu") (free yes) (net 4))
 (via (at 155.448 86.868) (size 0.8) (drill 0.4) (layers "F.Cu" "B.Cu") (free yes) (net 4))
 (via (at 155.194 94.234) (size 0.8) (drill 0.4) (layers "F.Cu" "B.Cu") (free yes) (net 4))
 (via (at 140.716 88.9) (size 0.8) (drill 0.4) (layers "F.Cu" "B.Cu") (free yes) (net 4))
 (via (at 154.178 104.648) (size 0.8) (drill 0.4) (layers "F.Cu" "B.Cu") (free yes) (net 4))
 (via (at 136.906 91.44) (size 0.8) (drill 0.4) (layers "F.Cu" "B.Cu") (free yes) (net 4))
 (via (at 155.5 100.75) (size 0.8) (drill 0.4) (layers "F.Cu" "B.Cu") (free yes) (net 4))
 (via (at 156.464 95.504) (size 0.8) (drill 0.4) (layers "F.Cu" "B.Cu") (free yes) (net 4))
 (via (at 140.716 91.44) (size 0.8) (drill 0.4) (layers "F.Cu" "B.Cu") (free yes) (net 4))
 (via (at 136.906 88.9) (size 0.8) (drill 0.4) (layers "F.Cu" "B.Cu") (free yes) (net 4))
 (via (at 142.24 93.726) (size 0.8) (drill 0.4) (layers "F.Cu" "B.Cu") (free yes) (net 4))
 (segment (start 145.5 95.8) (end 145.5 93) (width 0.21) (layer "F.Cu") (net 1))
 (segment (start 145.9 96.2) (end 147.762 96.2) (width 0.21) (layer "F.Cu") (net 6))
 (segment (start 150.114 97.236) (end 149 98.35) (width 0.5) (layer "F.Cu") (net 6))
 (segment (start 149.046 98.35) (end 149 98.35) (width 0.5) (layer "F.Cu") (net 6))
 (segment (start 148.082 86.614) (end 148.082 84.34852) (width 0.5) (layer "F.Cu") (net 6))
 (segment (start 149 97.438) (end 149 98.35) (width 0.21) (layer "F.Cu") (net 6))
 (segment (start 150.114 96.52) (end 150.114 97.236) (width 0.5) (layer "F.Cu") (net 6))
 (segment (start 147.762 96.2) (end 149 97.438) (width 0.21) (layer "F.Cu") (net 6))
 (via (at 150.114 96.52) (size 0.8) (drill 0.4) (layers "F.Cu" "B.Cu") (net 6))
 (segment (start 150.114 96.52) (end 150.114 88.646) (width 0.5) (layer "B.Cu") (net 6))
 (segment (start 150.114 88.646) (end 148.082 86.614) (width 0.5) (layer "B.Cu") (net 6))
 (segment (start 149 95.4125) (end 151.5 95.4125) (width 0.5) (layer "F.Cu") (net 2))
 (segment (start 151.5 95.4125) (end 151.5 98.35) (width 0.5) (layer "F.Cu") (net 2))
 (segment (start 145.9 95.8) (end 145.9 95.6) (width 0.21) (layer "F.Cu") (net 2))
 (segment (start 146.0875 95.4125) (end 149 95.4125) (width 0.21) (layer "F.Cu") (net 2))
 (segment (start 145.9 95.6) (end 146.0875 95.4125) (width 0.21) (layer "F.Cu") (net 2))
 (segment (start 145.5 96.2) (end 145.5 99) (width 0.21) (layer "F.Cu") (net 5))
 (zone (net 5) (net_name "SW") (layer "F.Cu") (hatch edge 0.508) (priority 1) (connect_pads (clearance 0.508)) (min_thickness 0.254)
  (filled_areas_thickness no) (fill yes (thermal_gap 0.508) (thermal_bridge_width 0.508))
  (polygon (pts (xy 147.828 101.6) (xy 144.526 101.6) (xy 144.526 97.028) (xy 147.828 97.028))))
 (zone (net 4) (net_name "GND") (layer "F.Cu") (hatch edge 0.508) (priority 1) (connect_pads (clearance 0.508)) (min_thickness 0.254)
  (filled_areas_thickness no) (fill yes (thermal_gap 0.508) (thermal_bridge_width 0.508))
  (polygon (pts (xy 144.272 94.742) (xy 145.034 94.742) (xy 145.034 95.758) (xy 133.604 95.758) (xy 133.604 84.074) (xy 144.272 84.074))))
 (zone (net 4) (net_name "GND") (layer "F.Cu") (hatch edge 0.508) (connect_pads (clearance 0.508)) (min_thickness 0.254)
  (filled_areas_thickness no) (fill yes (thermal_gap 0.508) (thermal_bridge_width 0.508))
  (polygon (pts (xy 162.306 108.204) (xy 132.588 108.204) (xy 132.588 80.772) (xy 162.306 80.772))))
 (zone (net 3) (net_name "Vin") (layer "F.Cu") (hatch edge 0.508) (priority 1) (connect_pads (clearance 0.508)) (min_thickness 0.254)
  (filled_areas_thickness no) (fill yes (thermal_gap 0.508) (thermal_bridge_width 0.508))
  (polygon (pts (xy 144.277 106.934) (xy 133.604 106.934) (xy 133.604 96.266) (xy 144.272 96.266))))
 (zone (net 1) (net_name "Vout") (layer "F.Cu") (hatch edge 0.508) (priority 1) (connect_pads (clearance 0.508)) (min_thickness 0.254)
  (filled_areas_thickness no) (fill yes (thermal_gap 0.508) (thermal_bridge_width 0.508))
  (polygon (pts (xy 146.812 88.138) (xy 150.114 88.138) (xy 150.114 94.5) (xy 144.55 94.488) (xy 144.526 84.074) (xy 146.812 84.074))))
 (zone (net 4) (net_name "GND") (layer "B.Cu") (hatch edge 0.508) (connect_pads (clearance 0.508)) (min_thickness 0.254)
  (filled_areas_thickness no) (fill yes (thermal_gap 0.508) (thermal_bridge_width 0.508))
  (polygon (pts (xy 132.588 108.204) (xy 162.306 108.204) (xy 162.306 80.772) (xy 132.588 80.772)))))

